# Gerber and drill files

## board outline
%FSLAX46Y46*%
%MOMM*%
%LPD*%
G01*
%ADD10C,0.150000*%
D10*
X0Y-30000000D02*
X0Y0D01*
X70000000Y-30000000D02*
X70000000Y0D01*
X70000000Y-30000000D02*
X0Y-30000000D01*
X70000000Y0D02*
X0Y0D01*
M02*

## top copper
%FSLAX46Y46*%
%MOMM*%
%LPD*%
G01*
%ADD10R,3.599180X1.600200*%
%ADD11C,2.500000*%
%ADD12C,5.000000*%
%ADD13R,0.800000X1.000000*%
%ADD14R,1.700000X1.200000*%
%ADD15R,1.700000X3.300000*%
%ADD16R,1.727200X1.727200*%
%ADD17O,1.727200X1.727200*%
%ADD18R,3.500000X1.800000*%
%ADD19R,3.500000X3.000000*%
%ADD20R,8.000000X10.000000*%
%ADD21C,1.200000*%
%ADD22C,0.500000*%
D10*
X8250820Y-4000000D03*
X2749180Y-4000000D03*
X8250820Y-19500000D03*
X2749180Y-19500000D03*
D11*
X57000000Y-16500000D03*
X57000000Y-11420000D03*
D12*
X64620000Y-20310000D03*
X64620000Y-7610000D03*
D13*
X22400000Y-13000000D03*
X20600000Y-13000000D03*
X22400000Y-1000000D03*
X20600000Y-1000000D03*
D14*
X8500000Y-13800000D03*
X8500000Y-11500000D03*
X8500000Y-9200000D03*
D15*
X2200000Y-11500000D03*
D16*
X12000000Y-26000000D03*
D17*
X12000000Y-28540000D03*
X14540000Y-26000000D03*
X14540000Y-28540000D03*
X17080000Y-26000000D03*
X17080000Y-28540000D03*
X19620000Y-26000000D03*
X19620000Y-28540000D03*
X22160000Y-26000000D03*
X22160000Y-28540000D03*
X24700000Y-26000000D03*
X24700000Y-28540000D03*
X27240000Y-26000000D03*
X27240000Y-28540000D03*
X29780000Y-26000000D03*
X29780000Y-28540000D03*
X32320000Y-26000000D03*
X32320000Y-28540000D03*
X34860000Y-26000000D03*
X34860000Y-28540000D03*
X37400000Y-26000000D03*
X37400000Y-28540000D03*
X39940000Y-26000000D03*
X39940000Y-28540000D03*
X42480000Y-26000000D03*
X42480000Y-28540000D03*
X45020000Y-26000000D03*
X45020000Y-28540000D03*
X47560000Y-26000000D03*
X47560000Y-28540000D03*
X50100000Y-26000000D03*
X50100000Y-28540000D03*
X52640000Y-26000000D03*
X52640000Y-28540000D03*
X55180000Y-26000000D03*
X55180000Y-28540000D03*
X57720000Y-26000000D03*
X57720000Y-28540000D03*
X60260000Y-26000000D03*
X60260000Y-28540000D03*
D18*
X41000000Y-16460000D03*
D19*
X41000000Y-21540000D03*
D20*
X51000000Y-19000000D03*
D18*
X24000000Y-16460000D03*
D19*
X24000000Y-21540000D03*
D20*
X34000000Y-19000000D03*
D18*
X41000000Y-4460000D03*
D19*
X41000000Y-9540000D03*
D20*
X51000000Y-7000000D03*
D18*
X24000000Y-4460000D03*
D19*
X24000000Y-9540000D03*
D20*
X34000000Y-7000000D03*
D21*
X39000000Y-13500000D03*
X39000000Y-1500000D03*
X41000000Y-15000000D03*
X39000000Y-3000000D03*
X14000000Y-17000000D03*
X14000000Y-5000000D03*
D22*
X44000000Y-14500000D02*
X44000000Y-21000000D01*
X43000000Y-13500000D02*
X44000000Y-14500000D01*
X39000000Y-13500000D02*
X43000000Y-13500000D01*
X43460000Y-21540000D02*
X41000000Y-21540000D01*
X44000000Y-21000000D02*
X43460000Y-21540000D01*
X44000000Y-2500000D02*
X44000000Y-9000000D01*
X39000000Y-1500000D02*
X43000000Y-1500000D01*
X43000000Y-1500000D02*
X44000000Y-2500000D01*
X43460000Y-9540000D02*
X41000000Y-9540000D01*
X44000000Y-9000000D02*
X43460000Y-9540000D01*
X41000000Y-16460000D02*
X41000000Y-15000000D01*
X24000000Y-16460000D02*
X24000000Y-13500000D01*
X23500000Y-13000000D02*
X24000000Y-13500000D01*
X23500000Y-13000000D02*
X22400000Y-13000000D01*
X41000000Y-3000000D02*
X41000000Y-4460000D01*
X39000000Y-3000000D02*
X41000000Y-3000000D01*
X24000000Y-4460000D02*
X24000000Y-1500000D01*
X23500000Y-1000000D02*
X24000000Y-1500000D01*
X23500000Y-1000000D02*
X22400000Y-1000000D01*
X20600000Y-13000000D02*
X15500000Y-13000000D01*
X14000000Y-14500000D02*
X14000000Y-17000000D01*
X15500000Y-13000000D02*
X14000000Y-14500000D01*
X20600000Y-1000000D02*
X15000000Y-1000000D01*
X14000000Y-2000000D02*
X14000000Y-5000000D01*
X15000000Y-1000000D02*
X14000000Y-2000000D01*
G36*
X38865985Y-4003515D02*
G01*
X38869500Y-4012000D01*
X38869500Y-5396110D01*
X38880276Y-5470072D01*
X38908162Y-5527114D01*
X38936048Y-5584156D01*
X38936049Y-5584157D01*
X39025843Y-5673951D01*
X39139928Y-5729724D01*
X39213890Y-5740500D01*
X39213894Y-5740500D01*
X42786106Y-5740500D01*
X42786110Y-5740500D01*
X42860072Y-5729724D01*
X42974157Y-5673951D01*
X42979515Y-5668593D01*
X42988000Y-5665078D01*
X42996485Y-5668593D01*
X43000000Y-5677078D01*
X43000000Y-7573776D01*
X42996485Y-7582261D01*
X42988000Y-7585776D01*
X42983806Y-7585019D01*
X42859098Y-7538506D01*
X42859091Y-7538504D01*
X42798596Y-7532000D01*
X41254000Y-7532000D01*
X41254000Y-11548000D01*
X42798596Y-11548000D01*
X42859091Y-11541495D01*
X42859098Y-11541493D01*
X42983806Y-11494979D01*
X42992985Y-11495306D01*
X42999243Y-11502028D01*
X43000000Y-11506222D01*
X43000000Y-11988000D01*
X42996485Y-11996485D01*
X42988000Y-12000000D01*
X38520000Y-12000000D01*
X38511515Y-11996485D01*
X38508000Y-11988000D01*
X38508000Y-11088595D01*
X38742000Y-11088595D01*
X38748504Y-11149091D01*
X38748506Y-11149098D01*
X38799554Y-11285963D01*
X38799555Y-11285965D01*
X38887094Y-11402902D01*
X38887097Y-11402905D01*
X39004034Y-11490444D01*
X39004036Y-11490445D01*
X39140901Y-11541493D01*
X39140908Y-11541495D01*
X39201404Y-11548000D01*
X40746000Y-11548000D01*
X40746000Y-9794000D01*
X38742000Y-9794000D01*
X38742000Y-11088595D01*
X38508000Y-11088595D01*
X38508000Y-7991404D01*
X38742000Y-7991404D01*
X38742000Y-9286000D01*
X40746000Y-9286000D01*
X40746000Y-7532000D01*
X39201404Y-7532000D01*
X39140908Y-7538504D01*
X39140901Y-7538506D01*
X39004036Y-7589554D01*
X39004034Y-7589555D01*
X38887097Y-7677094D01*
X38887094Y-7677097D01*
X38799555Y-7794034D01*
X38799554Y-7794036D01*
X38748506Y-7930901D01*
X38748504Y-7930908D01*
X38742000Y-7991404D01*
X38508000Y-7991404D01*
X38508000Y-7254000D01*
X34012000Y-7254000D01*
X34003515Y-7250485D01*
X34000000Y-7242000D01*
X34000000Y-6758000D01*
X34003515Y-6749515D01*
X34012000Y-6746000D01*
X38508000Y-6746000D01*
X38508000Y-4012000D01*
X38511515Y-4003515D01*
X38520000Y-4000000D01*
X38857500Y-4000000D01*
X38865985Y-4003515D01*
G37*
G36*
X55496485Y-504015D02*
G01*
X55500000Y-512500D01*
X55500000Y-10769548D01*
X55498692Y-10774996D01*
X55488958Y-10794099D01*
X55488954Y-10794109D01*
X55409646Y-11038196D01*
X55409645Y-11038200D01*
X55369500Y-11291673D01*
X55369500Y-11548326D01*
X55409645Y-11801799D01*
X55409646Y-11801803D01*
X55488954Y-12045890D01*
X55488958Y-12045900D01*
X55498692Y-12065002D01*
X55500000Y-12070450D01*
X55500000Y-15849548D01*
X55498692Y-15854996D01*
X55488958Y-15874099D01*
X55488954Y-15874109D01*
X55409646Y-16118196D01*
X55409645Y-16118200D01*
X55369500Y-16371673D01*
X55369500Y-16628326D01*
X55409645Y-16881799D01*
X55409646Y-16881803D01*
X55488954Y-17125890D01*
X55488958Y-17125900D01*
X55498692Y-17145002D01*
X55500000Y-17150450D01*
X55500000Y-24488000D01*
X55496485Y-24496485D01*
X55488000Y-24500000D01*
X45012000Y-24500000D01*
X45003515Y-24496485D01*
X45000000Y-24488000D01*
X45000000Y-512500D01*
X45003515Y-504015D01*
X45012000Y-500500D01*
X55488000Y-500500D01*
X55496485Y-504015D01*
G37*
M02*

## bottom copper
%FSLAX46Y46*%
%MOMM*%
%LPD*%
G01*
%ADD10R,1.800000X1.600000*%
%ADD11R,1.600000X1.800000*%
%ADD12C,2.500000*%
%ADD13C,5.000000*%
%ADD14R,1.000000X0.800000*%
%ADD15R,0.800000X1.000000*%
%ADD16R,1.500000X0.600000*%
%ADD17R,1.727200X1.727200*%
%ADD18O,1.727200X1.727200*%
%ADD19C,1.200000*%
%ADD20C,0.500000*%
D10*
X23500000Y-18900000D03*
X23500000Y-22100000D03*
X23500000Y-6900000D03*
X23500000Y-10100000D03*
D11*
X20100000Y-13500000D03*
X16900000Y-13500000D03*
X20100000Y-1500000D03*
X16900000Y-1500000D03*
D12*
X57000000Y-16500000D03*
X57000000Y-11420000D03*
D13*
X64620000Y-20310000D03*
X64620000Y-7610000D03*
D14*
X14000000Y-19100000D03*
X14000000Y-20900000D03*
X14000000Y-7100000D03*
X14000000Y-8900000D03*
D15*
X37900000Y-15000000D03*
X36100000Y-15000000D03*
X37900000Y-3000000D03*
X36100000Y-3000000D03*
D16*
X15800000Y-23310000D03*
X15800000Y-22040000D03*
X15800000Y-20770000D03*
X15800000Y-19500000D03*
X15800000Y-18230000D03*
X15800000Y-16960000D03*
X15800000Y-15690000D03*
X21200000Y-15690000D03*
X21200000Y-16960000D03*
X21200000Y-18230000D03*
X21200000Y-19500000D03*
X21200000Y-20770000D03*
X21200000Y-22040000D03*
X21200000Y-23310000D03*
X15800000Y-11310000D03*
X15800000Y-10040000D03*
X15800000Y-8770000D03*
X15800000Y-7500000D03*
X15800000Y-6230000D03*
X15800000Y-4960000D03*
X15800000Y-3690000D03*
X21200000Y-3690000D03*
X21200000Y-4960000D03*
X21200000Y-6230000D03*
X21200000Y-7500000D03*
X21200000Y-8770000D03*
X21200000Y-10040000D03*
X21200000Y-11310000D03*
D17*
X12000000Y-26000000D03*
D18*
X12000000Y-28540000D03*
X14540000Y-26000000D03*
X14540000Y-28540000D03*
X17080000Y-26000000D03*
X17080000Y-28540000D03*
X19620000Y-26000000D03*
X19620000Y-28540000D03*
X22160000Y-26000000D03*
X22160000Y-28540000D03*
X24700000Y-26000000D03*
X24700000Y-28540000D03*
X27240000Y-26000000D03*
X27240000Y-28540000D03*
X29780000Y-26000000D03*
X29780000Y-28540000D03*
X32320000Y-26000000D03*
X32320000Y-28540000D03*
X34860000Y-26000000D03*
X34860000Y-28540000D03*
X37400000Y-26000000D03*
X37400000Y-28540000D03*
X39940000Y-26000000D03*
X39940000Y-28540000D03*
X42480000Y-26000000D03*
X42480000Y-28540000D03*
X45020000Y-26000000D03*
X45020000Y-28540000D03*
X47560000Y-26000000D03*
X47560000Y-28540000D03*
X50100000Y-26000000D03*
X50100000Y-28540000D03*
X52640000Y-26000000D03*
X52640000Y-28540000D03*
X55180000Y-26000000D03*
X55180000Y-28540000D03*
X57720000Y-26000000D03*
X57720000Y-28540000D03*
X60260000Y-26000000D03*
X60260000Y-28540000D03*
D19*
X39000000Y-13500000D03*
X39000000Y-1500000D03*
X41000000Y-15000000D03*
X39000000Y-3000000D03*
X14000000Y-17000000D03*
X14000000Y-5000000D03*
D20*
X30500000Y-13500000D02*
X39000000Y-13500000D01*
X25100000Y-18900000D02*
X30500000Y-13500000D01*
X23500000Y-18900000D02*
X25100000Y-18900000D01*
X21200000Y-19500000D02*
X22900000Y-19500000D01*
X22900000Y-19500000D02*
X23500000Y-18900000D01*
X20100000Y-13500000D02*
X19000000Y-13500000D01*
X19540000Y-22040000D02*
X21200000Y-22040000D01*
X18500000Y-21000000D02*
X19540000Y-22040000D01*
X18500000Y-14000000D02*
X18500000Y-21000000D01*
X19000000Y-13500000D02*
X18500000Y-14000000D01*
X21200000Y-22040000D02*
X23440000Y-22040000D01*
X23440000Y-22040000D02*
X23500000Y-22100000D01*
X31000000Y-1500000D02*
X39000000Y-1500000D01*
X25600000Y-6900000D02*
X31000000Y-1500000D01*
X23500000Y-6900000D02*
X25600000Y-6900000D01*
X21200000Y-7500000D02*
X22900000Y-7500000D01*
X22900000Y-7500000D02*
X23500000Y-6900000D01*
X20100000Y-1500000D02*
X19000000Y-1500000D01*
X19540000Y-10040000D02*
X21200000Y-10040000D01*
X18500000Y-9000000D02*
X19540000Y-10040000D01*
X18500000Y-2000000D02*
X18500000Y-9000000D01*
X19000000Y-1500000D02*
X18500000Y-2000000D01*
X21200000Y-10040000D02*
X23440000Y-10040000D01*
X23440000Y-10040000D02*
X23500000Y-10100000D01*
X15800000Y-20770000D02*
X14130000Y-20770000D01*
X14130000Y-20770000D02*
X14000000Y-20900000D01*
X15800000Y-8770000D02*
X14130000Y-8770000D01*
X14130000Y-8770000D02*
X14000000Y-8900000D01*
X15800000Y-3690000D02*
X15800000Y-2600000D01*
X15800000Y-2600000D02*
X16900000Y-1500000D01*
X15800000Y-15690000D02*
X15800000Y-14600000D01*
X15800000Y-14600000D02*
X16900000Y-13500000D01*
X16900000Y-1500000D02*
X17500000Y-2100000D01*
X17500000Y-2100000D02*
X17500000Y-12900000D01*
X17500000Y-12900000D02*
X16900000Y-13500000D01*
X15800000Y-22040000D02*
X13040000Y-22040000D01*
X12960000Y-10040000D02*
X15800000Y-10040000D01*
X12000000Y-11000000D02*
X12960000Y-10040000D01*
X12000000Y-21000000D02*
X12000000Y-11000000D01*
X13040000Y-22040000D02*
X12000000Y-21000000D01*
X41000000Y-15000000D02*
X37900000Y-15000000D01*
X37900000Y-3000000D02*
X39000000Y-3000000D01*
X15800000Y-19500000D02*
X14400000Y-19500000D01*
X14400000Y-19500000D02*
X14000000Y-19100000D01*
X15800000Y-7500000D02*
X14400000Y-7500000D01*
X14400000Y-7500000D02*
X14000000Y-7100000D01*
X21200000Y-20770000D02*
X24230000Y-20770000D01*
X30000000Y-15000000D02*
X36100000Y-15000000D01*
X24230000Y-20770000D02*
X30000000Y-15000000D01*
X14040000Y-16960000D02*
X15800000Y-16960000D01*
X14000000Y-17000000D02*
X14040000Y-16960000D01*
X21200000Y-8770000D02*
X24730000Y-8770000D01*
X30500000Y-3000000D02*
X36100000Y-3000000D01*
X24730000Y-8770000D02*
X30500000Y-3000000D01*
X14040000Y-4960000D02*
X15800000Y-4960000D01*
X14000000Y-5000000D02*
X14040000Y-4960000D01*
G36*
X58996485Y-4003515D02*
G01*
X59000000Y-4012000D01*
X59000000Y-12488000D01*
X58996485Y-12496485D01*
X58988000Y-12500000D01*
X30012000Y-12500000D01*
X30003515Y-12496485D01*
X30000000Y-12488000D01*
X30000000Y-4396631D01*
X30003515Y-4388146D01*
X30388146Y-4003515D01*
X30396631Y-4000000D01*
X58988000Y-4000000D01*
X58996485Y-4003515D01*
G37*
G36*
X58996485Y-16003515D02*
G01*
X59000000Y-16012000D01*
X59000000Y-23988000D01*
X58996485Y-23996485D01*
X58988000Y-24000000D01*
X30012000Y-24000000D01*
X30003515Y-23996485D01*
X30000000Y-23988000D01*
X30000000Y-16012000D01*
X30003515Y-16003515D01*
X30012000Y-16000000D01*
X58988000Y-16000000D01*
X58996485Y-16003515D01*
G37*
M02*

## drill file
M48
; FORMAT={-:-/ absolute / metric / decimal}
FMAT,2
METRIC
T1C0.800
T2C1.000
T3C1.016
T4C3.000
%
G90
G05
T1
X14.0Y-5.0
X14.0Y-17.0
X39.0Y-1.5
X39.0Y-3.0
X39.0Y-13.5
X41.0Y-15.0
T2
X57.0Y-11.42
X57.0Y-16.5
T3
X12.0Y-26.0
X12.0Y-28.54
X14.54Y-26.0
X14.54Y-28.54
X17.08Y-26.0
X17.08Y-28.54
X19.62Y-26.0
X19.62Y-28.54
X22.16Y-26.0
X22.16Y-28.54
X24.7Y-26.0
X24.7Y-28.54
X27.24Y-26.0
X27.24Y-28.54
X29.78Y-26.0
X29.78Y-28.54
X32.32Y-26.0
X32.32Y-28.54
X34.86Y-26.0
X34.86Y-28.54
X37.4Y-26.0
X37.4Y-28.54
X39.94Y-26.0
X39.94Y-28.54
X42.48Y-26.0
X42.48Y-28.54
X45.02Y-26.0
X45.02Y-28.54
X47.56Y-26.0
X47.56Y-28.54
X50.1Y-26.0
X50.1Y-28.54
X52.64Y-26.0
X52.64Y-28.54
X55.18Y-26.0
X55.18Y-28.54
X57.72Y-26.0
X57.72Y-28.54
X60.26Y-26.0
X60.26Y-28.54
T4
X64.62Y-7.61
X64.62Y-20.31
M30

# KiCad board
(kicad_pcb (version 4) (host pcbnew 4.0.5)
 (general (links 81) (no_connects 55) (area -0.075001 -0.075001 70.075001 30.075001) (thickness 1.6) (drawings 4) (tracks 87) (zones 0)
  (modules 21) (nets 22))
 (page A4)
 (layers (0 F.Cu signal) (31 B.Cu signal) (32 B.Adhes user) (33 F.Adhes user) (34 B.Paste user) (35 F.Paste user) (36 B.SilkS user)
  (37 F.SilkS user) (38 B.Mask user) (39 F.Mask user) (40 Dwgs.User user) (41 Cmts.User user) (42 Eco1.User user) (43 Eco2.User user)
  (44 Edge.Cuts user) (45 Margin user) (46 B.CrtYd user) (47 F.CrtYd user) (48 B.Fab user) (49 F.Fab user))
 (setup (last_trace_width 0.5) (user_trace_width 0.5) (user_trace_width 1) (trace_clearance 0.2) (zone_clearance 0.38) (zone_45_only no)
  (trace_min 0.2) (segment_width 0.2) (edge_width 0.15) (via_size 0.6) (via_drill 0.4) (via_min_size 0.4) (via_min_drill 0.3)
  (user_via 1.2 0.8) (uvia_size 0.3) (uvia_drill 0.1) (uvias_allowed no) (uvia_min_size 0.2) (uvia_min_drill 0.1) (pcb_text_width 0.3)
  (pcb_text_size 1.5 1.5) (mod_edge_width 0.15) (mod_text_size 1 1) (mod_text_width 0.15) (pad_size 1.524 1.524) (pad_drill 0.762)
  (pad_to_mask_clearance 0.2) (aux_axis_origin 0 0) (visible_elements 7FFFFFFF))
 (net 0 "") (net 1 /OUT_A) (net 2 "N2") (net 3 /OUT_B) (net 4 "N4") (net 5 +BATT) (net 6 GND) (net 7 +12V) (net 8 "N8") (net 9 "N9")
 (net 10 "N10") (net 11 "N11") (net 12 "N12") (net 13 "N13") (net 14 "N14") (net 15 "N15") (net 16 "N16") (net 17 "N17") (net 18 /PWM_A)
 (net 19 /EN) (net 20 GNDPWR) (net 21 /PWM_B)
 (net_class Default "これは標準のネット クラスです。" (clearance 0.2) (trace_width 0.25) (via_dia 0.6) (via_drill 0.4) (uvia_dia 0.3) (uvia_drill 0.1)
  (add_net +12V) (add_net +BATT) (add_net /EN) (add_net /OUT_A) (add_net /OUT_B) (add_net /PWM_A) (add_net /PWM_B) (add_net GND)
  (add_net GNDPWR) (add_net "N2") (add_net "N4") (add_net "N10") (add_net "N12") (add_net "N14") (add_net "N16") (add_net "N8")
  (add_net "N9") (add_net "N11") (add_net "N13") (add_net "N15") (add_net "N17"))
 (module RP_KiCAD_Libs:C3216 (layer B.Cu) (at 23.5 20.5 270)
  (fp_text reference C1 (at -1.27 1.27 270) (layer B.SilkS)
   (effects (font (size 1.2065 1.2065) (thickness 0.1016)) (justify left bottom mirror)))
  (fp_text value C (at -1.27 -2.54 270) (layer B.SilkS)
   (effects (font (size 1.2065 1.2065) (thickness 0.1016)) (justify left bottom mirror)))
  (pad 1 smd rect (at -1.6 0 270) (size 1.6 1.8) (layers B.Cu B.Paste B.Mask) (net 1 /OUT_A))
  (pad 2 smd rect (at 1.6 0 270) (size 1.6 1.8) (layers B.Cu B.Paste B.Mask) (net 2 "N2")))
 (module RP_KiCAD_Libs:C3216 (layer B.Cu) (at 23.5 8.5 270)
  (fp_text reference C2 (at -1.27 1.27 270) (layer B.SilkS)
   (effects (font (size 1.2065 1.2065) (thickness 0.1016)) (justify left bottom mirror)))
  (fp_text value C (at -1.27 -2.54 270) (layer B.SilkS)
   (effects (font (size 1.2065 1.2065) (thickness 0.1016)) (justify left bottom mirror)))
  (pad 1 smd rect (at -1.6 0 270) (size 1.6 1.8) (layers B.Cu B.Paste B.Mask) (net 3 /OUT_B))
  (pad 2 smd rect (at 1.6 0 270) (size 1.6 1.8) (layers B.Cu B.Paste B.Mask) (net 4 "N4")))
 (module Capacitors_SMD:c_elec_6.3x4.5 (layer F.Cu) (at 5.5 4)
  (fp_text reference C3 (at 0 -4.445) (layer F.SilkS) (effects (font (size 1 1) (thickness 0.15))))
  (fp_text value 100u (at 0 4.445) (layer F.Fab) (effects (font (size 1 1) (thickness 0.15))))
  (pad 1 smd rect (at 2.75082 0) (size 3.59918 1.6002) (layers F.Cu F.Paste F.Mask) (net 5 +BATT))
  (pad 2 smd rect (at -2.75082 0) (size 3.59918 1.6002) (layers F.Cu F.Paste F.Mask) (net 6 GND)))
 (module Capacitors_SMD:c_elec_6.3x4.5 (layer F.Cu) (at 5.5 19.5)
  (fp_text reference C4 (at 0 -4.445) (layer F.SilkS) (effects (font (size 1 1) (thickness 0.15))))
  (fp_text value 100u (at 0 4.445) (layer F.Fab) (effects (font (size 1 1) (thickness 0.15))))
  (pad 1 smd rect (at 2.75082 0) (size 3.59918 1.6002) (layers F.Cu F.Paste F.Mask) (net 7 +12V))
  (pad 2 smd rect (at -2.75082 0) (size 3.59918 1.6002) (layers F.Cu F.Paste F.Mask) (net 6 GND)))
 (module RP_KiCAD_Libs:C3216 (layer B.Cu) (at 18.5 13.5 180)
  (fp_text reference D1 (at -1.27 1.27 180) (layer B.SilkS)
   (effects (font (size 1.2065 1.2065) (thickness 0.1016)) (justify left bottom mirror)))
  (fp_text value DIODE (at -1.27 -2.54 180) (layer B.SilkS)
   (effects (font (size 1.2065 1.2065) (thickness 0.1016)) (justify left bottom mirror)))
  (pad 1 smd rect (at -1.6 0 180) (size 1.6 1.8) (layers B.Cu B.Paste B.Mask) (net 2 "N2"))
  (pad 2 smd rect (at 1.6 0 180) (size 1.6 1.8) (layers B.Cu B.Paste B.Mask) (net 7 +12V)))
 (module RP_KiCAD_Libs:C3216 (layer B.Cu) (at 18.5 1.5 180)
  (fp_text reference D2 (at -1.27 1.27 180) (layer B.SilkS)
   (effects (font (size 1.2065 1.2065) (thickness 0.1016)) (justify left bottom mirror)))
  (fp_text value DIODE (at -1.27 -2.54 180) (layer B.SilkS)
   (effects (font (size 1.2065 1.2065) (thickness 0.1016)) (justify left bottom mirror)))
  (pad 1 smd rect (at -1.6 0 180) (size 1.6 1.8) (layers B.Cu B.Paste B.Mask) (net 4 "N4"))
  (pad 2 smd rect (at 1.6 0 180) (size 1.6 1.8) (layers B.Cu B.Paste B.Mask) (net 7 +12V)))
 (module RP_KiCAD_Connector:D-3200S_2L (layer F.Cu) (at 57 16.5 90)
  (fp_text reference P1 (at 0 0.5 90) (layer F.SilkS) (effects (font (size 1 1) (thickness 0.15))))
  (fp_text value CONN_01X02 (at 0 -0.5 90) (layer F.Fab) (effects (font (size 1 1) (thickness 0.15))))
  (pad 1 thru_hole circle (at 0 0 90) (size 2.5 2.5) (drill 1) (layers *.Cu *.Mask F.SilkS) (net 1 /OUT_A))
  (pad 2 thru_hole circle (at 5.08 0 90) (size 2.5 2.5) (drill 1) (layers *.Cu *.Mask F.SilkS) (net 3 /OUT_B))
  (pad "" thru_hole circle (at -3.81 7.62 90) (size 5 5) (drill 3) (layers *.Cu *.Mask F.SilkS))
  (pad "" thru_hole circle (at 8.89 7.62 90) (size 5 5) (drill 3) (layers *.Cu *.Mask F.SilkS)))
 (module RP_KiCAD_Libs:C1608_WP (layer B.Cu) (at 14 20 270)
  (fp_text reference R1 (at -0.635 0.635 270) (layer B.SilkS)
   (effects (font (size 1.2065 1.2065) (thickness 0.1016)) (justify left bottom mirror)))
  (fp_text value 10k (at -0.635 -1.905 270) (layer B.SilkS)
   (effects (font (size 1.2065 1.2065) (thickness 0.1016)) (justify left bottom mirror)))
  (pad 1 smd rect (at -0.9 0 270) (size 0.8 1) (layers B.Cu B.Paste B.Mask) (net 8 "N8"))
  (pad 2 smd rect (at 0.9 0 270) (size 0.8 1) (layers B.Cu B.Paste B.Mask) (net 6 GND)))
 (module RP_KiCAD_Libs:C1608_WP (layer B.Cu) (at 14 8 270)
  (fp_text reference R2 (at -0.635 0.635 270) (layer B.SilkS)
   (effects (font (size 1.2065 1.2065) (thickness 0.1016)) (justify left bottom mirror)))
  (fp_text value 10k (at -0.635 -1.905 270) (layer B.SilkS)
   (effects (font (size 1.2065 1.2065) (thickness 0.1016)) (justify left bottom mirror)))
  (pad 1 smd rect (at -0.9 0 270) (size 0.8 1) (layers B.Cu B.Paste B.Mask) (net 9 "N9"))
  (pad 2 smd rect (at 0.9 0 270) (size 0.8 1) (layers B.Cu B.Paste B.Mask) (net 6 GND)))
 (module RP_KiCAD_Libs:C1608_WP (layer B.Cu) (at 37 15 180)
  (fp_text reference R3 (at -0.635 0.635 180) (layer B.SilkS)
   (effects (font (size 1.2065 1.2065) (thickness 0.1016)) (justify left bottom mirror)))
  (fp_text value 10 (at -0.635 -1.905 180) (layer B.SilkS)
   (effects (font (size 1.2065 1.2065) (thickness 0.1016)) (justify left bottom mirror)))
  (pad 1 smd rect (at -0.9 0 180) (size 0.8 1) (layers B.Cu B.Paste B.Mask) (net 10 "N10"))
  (pad 2 smd rect (at 0.9 0 180) (size 0.8 1) (layers B.Cu B.Paste B.Mask) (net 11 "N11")))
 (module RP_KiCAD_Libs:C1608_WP (layer F.Cu) (at 21.5 13 180)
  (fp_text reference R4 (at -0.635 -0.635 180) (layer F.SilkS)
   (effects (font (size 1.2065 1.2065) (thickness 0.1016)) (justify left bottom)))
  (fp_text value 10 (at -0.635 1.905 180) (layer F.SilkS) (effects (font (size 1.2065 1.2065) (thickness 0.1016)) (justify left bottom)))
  (pad 1 smd rect (at -0.9 0 180) (size 0.8 1) (layers F.Cu F.Paste F.Mask) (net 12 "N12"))
  (pad 2 smd rect (at 0.9 0 180) (size 0.8 1) (layers F.Cu F.Paste F.Mask) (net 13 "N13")))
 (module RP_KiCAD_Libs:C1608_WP (layer B.Cu) (at 37 3 180)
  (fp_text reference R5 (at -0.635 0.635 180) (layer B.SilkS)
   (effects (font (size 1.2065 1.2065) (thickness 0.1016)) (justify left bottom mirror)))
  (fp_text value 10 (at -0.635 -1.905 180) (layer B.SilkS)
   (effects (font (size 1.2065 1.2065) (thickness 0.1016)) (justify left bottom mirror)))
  (pad 1 smd rect (at -0.9 0 180) (size 0.8 1) (layers B.Cu B.Paste B.Mask) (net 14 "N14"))
  (pad 2 smd rect (at 0.9 0 180) (size 0.8 1) (layers B.Cu B.Paste B.Mask) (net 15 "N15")))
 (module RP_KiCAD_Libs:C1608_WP (layer F.Cu) (at 21.5 1 180)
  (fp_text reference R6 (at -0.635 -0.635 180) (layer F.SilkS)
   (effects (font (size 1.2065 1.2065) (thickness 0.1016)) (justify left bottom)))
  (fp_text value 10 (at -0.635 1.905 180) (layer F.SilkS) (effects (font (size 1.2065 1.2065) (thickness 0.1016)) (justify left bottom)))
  (pad 1 smd rect (at -0.9 0 180) (size 0.8 1) (layers F.Cu F.Paste F.Mask) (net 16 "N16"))
  (pad 2 smd rect (at 0.9 0 180) (size 0.8 1) (layers F.Cu F.Paste F.Mask) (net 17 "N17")))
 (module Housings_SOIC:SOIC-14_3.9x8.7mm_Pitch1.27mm (layer B.Cu) (at 18.5 19.5)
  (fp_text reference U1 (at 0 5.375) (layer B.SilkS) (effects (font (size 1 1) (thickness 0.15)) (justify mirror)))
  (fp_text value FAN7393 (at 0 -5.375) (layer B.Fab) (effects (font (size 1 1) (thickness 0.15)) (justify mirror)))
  (pad 1 smd rect (at -2.7 3.81) (size 1.5 0.6) (layers B.Cu B.Paste B.Mask) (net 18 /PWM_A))
  (pad 2 smd rect (at -2.7 2.54) (size 1.5 0.6) (layers B.Cu B.Paste B.Mask) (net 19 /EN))
  (pad 3 smd rect (at -2.7 1.27) (size 1.5 0.6) (layers B.Cu B.Paste B.Mask) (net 6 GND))
  (pad 4 smd rect (at -2.7 0) (size 1.5 0.6) (layers B.Cu B.Paste B.Mask) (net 8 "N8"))
  (pad 5 smd rect (at -2.7 -1.27) (size 1.5 0.6) (layers B.Cu B.Paste B.Mask) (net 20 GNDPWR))
  (pad 6 smd rect (at -2.7 -2.54) (size 1.5 0.6) (layers B.Cu B.Paste B.Mask) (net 13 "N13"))
  (pad 7 smd rect (at -2.7 -3.81) (size 1.5 0.6) (layers B.Cu B.Paste B.Mask) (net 7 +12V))
  (pad 8 smd rect (at 2.7 -3.81) (size 1.5 0.6) (layers B.Cu B.Paste B.Mask))
  (pad 9 smd rect (at 2.7 -2.54) (size 1.5 0.6) (layers B.Cu B.Paste B.Mask))
  (pad 10 smd rect (at 2.7 -1.27) (size 1.5 0.6) (layers B.Cu B.Paste B.Mask))
  (pad 11 smd rect (at 2.7 0) (size 1.5 0.6) (layers B.Cu B.Paste B.Mask) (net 1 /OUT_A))
  (pad 12 smd rect (at 2.7 1.27) (size 1.5 0.6) (layers B.Cu B.Paste B.Mask) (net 11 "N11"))
  (pad 13 smd rect (at 2.7 2.54) (size 1.5 0.6) (layers B.Cu B.Paste B.Mask) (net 2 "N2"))
  (pad 14 smd rect (at 2.7 3.81) (size 1.5 0.6) (layers B.Cu B.Paste B.Mask)))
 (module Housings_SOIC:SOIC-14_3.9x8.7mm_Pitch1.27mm (layer B.Cu) (at 18.5 7.5)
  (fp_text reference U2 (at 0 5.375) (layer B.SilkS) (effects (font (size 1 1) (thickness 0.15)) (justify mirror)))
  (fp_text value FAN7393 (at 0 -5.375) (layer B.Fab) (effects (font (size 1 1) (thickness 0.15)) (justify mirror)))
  (pad 1 smd rect (at -2.7 3.81) (size 1.5 0.6) (layers B.Cu B.Paste B.Mask) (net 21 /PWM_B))
  (pad 2 smd rect (at -2.7 2.54) (size 1.5 0.6) (layers B.Cu B.Paste B.Mask) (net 19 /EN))
  (pad 3 smd rect (at -2.7 1.27) (size 1.5 0.6) (layers B.Cu B.Paste B.Mask) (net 6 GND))
  (pad 4 smd rect (at -2.7 0) (size 1.5 0.6) (layers B.Cu B.Paste B.Mask) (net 9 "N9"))
  (pad 5 smd rect (at -2.7 -1.27) (size 1.5 0.6) (layers B.Cu B.Paste B.Mask) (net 20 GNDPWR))
  (pad 6 smd rect (at -2.7 -2.54) (size 1.5 0.6) (layers B.Cu B.Paste B.Mask) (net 17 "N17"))
  (pad 7 smd rect (at -2.7 -3.81) (size 1.5 0.6) (layers B.Cu B.Paste B.Mask) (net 7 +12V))
  (pad 8 smd rect (at 2.7 -3.81) (size 1.5 0.6) (layers B.Cu B.Paste B.Mask))
  (pad 9 smd rect (at 2.7 -2.54) (size 1.5 0.6) (layers B.Cu B.Paste B.Mask))
  (pad 10 smd rect (at 2.7 -1.27) (size 1.5 0.6) (layers B.Cu B.Paste B.Mask))
  (pad 11 smd rect (at 2.7 0) (size 1.5 0.6) (layers B.Cu B.Paste B.Mask) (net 3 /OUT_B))
  (pad 12 smd rect (at 2.7 1.27) (size 1.5 0.6) (layers B.Cu B.Paste B.Mask) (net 15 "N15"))
  (pad 13 smd rect (at 2.7 2.54) (size 1.5 0.6) (layers B.Cu B.Paste B.Mask) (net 4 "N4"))
  (pad 14 smd rect (at 2.7 3.81) (size 1.5 0.6) (layers B.Cu B.Paste B.Mask)))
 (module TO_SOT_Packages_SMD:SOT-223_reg (layer F.Cu) (at 8.5 11.5 90)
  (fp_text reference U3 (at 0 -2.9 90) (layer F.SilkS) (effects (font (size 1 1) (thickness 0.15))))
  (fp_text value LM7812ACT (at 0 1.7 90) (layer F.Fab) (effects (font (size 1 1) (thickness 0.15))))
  (pad 1 smd rect (at -2.3 0 90) (size 1.2 1.7) (layers F.Cu F.Paste F.Mask) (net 5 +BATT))
  (pad 2 smd rect (at 0 0 90) (size 1.2 1.7) (layers F.Cu F.Paste F.Mask) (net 6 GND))
  (pad 3 smd rect (at 2.3 0 90) (size 1.2 1.7) (layers F.Cu F.Paste F.Mask) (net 7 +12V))
  (pad 2 smd rect (at 0 -6.3 90) (size 3.3 1.7) (layers F.Cu F.Paste F.Mask) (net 6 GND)))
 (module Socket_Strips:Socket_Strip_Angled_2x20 (layer F.Cu) (at 12 26)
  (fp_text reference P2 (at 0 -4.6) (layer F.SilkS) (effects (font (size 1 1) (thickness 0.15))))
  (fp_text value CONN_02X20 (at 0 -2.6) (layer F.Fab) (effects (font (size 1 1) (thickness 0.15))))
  (pad 1 thru_hole rect (at 0 0) (size 1.7272 1.7272) (drill 1.016) (layers *.Cu *.Mask F.SilkS) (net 6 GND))
  (pad 2 thru_hole oval (at 0 2.54) (size 1.7272 1.7272) (drill 1.016) (layers *.Cu *.Mask F.SilkS) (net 21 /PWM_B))
  (pad 3 thru_hole oval (at 2.54 0) (size 1.7272 1.7272) (drill 1.016) (layers *.Cu *.Mask F.SilkS) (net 19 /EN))
  (pad 4 thru_hole oval (at 2.54 2.54) (size 1.7272 1.7272) (drill 1.016) (layers *.Cu *.Mask F.SilkS) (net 18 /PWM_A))
  (pad 5 thru_hole oval (at 5.08 0) (size 1.7272 1.7272) (drill 1.016) (layers *.Cu *.Mask F.SilkS) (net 20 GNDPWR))
  (pad 6 thru_hole oval (at 5.08 2.54) (size 1.7272 1.7272) (drill 1.016) (layers *.Cu *.Mask F.SilkS) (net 20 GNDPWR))
  (pad 7 thru_hole oval (at 7.62 0) (size 1.7272 1.7272) (drill 1.016) (layers *.Cu *.Mask F.SilkS) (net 20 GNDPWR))
  (pad 8 thru_hole oval (at 7.62 2.54) (size 1.7272 1.7272) (drill 1.016) (layers *.Cu *.Mask F.SilkS) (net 20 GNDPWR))
  (pad 9 thru_hole oval (at 10.16 0) (size 1.7272 1.7272) (drill 1.016) (layers *.Cu *.Mask F.SilkS) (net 20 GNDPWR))
  (pad 10 thru_hole oval (at 10.16 2.54) (size 1.7272 1.7272) (drill 1.016) (layers *.Cu *.Mask F.SilkS) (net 20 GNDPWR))
  (pad 11 thru_hole oval (at 12.7 0) (size 1.7272 1.7272) (drill 1.016) (layers *.Cu *.Mask F.SilkS) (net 20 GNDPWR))
  (pad 12 thru_hole oval (at 12.7 2.54) (size 1.7272 1.7272) (drill 1.016) (layers *.Cu *.Mask F.SilkS) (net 20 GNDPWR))
  (pad 13 thru_hole oval (at 15.24 0) (size 1.7272 1.7272) (drill 1.016) (layers *.Cu *.Mask F.SilkS) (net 20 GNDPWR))
  (pad 14 thru_hole oval (at 15.24 2.54) (size 1.7272 1.7272) (drill 1.016) (layers *.Cu *.Mask F.SilkS) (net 20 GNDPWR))
  (pad 15 thru_hole oval (at 17.78 0) (size 1.7272 1.7272) (drill 1.016) (layers *.Cu *.Mask F.SilkS) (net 20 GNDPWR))
  (pad 16 thru_hole oval (at 17.78 2.54) (size 1.7272 1.7272) (drill 1.016) (layers *.Cu *.Mask F.SilkS) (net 20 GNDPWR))
  (pad 17 thru_hole oval (at 20.32 0) (size 1.7272 1.7272) (drill 1.016) (layers *.Cu *.Mask F.SilkS) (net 20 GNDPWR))
  (pad 18 thru_hole oval (at 20.32 2.54) (size 1.7272 1.7272) (drill 1.016) (layers *.Cu *.Mask F.SilkS) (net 20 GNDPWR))
  (pad 19 thru_hole oval (at 22.86 0) (size 1.7272 1.7272) (drill 1.016) (layers *.Cu *.Mask F.SilkS) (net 20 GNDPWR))
  (pad 20 thru_hole oval (at 22.86 2.54) (size 1.7272 1.7272) (drill 1.016) (layers *.Cu *.Mask F.SilkS) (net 20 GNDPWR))
  (pad 21 thru_hole oval (at 25.4 0) (size 1.7272 1.7272) (drill 1.016) (layers *.Cu *.Mask F.SilkS) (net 20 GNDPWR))
  (pad 22 thru_hole oval (at 25.4 2.54) (size 1.7272 1.7272) (drill 1.016) (layers *.Cu *.Mask F.SilkS) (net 20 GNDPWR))
  (pad 23 thru_hole oval (at 27.94 0) (size 1.7272 1.7272) (drill 1.016) (layers *.Cu *.Mask F.SilkS) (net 5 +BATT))
  (pad 24 thru_hole oval (at 27.94 2.54) (size 1.7272 1.7272) (drill 1.016) (layers *.Cu *.Mask F.SilkS) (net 5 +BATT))
  (pad 25 thru_hole oval (at 30.48 0) (size 1.7272 1.7272) (drill 1.016) (layers *.Cu *.Mask F.SilkS) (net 5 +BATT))
  (pad 26 thru_hole oval (at 30.48 2.54) (size 1.7272 1.7272) (drill 1.016) (layers *.Cu *.Mask F.SilkS) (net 5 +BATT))
  (pad 27 thru_hole oval (at 33.02 0) (size 1.7272 1.7272) (drill 1.016) (layers *.Cu *.Mask F.SilkS) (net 5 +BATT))
  (pad 28 thru_hole oval (at 33.02 2.54) (size 1.7272 1.7272) (drill 1.016) (layers *.Cu *.Mask F.SilkS) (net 5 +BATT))
  (pad 29 thru_hole oval (at 35.56 0) (size 1.7272 1.7272) (drill 1.016) (layers *.Cu *.Mask F.SilkS) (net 5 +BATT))
  (pad 30 thru_hole oval (at 35.56 2.54) (size 1.7272 1.7272) (drill 1.016) (layers *.Cu *.Mask F.SilkS) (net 5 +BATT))
  (pad 31 thru_hole oval (at 38.1 0) (size 1.7272 1.7272) (drill 1.016) (layers *.Cu *.Mask F.SilkS) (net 5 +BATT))
  (pad 32 thru_hole oval (at 38.1 2.54) (size 1.7272 1.7272) (drill 1.016) (layers *.Cu *.Mask F.SilkS) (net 5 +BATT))
  (pad 33 thru_hole oval (at 40.64 0) (size 1.7272 1.7272) (drill 1.016) (layers *.Cu *.Mask F.SilkS) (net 5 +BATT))
  (pad 34 thru_hole oval (at 40.64 2.54) (size 1.7272 1.7272) (drill 1.016) (layers *.Cu *.Mask F.SilkS) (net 5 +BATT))
  (pad 35 thru_hole oval (at 43.18 0) (size 1.7272 1.7272) (drill 1.016) (layers *.Cu *.Mask F.SilkS) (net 5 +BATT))
  (pad 36 thru_hole oval (at 43.18 2.54) (size 1.7272 1.7272) (drill 1.016) (layers *.Cu *.Mask F.SilkS) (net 5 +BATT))
  (pad 37 thru_hole oval (at 45.72 0) (size 1.7272 1.7272) (drill 1.016) (layers *.Cu *.Mask F.SilkS) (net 5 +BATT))
  (pad 38 thru_hole oval (at 45.72 2.54) (size 1.7272 1.7272) (drill 1.016) (layers *.Cu *.Mask F.SilkS) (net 5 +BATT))
  (pad 39 thru_hole oval (at 48.26 0) (size 1.7272 1.7272) (drill 1.016) (layers *.Cu *.Mask F.SilkS) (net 5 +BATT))
  (pad 40 thru_hole oval (at 48.26 2.54) (size 1.7272 1.7272) (drill 1.016) (layers *.Cu *.Mask F.SilkS) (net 5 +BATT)))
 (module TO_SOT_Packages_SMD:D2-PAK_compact (layer F.Cu) (at 44 19 270)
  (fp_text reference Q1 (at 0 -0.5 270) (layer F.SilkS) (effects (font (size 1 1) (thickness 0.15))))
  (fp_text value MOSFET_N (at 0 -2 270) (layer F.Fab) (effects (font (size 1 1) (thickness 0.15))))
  (pad G smd rect (at -2.54 3 270) (size 1.8 3.5) (layers F.Cu F.Paste F.Mask) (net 10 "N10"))
  (pad S smd rect (at 2.54 3 270) (size 3 3.5) (layers F.Cu F.Paste F.Mask) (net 1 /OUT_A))
  (pad D smd rect (at 0 -7 270) (size 10 8) (layers F.Cu F.Paste F.Mask) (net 5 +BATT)))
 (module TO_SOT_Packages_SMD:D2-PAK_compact (layer F.Cu) (at 27 19 270)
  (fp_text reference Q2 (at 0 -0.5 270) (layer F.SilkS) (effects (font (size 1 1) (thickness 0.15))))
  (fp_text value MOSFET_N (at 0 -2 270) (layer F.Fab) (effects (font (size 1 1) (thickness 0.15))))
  (pad G smd rect (at -2.54 3 270) (size 1.8 3.5) (layers F.Cu F.Paste F.Mask) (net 12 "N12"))
  (pad S smd rect (at 2.54 3 270) (size 3 3.5) (layers F.Cu F.Paste F.Mask) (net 20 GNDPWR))
  (pad D smd rect (at 0 -7 270) (size 10 8) (layers F.Cu F.Paste F.Mask) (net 1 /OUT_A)))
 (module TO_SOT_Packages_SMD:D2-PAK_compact (layer F.Cu) (at 44 7 270)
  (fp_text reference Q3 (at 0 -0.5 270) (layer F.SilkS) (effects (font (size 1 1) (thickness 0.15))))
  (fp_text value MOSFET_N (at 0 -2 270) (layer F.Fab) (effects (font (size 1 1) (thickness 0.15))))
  (pad G smd rect (at -2.54 3 270) (size 1.8 3.5) (layers F.Cu F.Paste F.Mask) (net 14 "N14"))
  (pad S smd rect (at 2.54 3 270) (size 3 3.5) (layers F.Cu F.Paste F.Mask) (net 3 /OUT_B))
  (pad D smd rect (at 0 -7 270) (size 10 8) (layers F.Cu F.Paste F.Mask) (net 5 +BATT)))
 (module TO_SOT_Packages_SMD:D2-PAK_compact (layer F.Cu) (at 27 7 270)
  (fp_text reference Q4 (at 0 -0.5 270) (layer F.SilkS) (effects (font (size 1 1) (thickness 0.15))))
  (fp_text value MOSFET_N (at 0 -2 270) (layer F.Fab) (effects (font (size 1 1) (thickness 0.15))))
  (pad G smd rect (at -2.54 3 270) (size 1.8 3.5) (layers F.Cu F.Paste F.Mask) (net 16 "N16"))
  (pad S smd rect (at 2.54 3 270) (size 3 3.5) (layers F.Cu F.Paste F.Mask) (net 20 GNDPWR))
  (pad D smd rect (at 0 -7 270) (size 10 8) (layers F.Cu F.Paste F.Mask) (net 3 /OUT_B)))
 (gr_line (start 0 30) (end 0 0) (angle 90) (layer Edge.Cuts) (width 0.15))
 (gr_line (start 70 30) (end 70 0) (angle 90) (layer Edge.Cuts) (width 0.15))
 (gr_line (start 70 30) (end 0 30) (angle 90) (layer Edge.Cuts) (width 0.15))
 (gr_line (start 70 0) (end 0 0) (angle 90) (layer Edge.Cuts) (width 0.15))
 (segment (start 44 14.5) (end 44 21) (width 0.5) (layer F.Cu) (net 1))
 (segment (start 43 13.5) (end 44 14.5) (width 0.5) (layer F.Cu) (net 1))
 (segment (start 39 13.5) (end 43 13.5) (width 0.5) (layer F.Cu) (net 1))
 (via (at 39 13.5) (size 1.2) (drill 0.8) (layers F.Cu B.Cu) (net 1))
 (segment (start 30.5 13.5) (end 39 13.5) (width 0.5) (layer B.Cu) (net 1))
 (segment (start 25.1 18.9) (end 30.5 13.5) (width 0.5) (layer B.Cu) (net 1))
 (segment (start 23.5 18.9) (end 25.1 18.9) (width 0.5) (layer B.Cu) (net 1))
 (segment (start 43.46 21.54) (end 41 21.54) (width 0.5) (layer F.Cu) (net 1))
 (segment (start 44 21) (end 43.46 21.54) (width 0.5) (layer F.Cu) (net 1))
 (segment (start 21.2 19.5) (end 22.9 19.5) (width 0.5) (layer B.Cu) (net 1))
 (segment (start 22.9 19.5) (end 23.5 18.9) (width 0.5) (layer B.Cu) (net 1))
 (segment (start 20.1 13.5) (end 19 13.5) (width 0.5) (layer B.Cu) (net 2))
 (segment (start 19.54 22.04) (end 21.2 22.04) (width 0.5) (layer B.Cu) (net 2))
 (segment (start 18.5 21) (end 19.54 22.04) (width 0.5) (layer B.Cu) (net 2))
 (segment (start 18.5 14) (end 18.5 21) (width 0.5) (layer B.Cu) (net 2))
 (segment (start 19 13.5) (end 18.5 14) (width 0.5) (layer B.Cu) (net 2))
 (segment (start 21.2 22.04) (end 23.44 22.04) (width 0.5) (layer B.Cu) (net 2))
 (segment (start 23.44 22.04) (end 23.5 22.1) (width 0.5) (layer B.Cu) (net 2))
 (segment (start 44 2.5) (end 44 9) (width 0.5) (layer F.Cu) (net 3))
 (via (at 39 1.5) (size 1.2) (drill 0.8) (layers F.Cu B.Cu) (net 3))
 (segment (start 39 1.5) (end 43 1.5) (width 0.5) (layer F.Cu) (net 3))
 (segment (start 43 1.5) (end 44 2.5) (width 0.5) (layer F.Cu) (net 3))
 (segment (start 31 1.5) (end 39 1.5) (width 0.5) (layer B.Cu) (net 3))
 (segment (start 25.6 6.9) (end 31 1.5) (width 0.5) (layer B.Cu) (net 3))
 (segment (start 23.5 6.9) (end 25.6 6.9) (width 0.5) (layer B.Cu) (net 3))
 (segment (start 43.46 9.54) (end 41 9.54) (width 0.5) (layer F.Cu) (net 3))
 (segment (start 44 9) (end 43.46 9.54) (width 0.5) (layer F.Cu) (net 3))
 (segment (start 21.2 7.5) (end 22.9 7.5) (width 0.5) (layer B.Cu) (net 3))
 (segment (start 22.9 7.5) (end 23.5 6.9) (width 0.5) (layer B.Cu) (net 3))
 (segment (start 20.1 1.5) (end 19 1.5) (width 0.5) (layer B.Cu) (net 4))
 (segment (start 19.54 10.04) (end 21.2 10.04) (width 0.5) (layer B.Cu) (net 4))
 (segment (start 18.5 9) (end 19.54 10.04) (width 0.5) (layer B.Cu) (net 4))
 (segment (start 18.5 2) (end 18.5 9) (width 0.5) (layer B.Cu) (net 4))
 (segment (start 19 1.5) (end 18.5 2) (width 0.5) (layer B.Cu) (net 4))
 (segment (start 21.2 10.04) (end 23.44 10.04) (width 0.5) (layer B.Cu) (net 4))
 (segment (start 23.44 10.04) (end 23.5 10.1) (width 0.5) (layer B.Cu) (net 4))
 (segment (start 15.8 20.77) (end 14.13 20.77) (width 0.5) (layer B.Cu) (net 6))
 (segment (start 14.13 20.77) (end 14 20.9) (width 0.5) (layer B.Cu) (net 6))
 (segment (start 15.8 8.77) (end 14.13 8.77) (width 0.5) (layer B.Cu) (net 6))
 (segment (start 14.13 8.77) (end 14 8.9) (width 0.5) (layer B.Cu) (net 6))
 (segment (start 15.8 3.69) (end 15.8 2.6) (width 0.5) (layer B.Cu) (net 7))
 (segment (start 15.8 2.6) (end 16.9 1.5) (width 0.5) (layer B.Cu) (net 7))
 (segment (start 15.8 15.69) (end 15.8 14.6) (width 0.5) (layer B.Cu) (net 7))
 (segment (start 15.8 14.6) (end 16.9 13.5) (width 0.5) (layer B.Cu) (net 7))
 (segment (start 16.9 1.5) (end 17.5 2.1) (width 0.5) (layer B.Cu) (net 7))
 (segment (start 17.5 2.1) (end 17.5 12.9) (width 0.5) (layer B.Cu) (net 7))
 (segment (start 17.5 12.9) (end 16.9 13.5) (width 0.5) (layer B.Cu) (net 7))
 (segment (start 15.8 22.04) (end 13.04 22.04) (width 0.5) (layer B.Cu) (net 19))
 (segment (start 12.96 10.04) (end 15.8 10.04) (width 0.5) (layer B.Cu) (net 19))
 (segment (start 12 11) (end 12.96 10.04) (width 0.5) (layer B.Cu) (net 19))
 (segment (start 12 21) (end 12 11) (width 0.5) (layer B.Cu) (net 19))
 (segment (start 13.04 22.04) (end 12 21) (width 0.5) (layer B.Cu) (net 19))
 (segment (start 41 16.46) (end 41 15) (width 0.5) (layer F.Cu) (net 10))
 (segment (start 41 15) (end 37.9 15) (width 0.5) (layer B.Cu) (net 10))
 (via (at 41 15) (size 1.2) (drill 0.8) (layers F.Cu B.Cu) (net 10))
 (segment (start 24 16.46) (end 24 13.5) (width 0.5) (layer F.Cu) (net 12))
 (segment (start 23.5 13) (end 24 13.5) (width 0.5) (layer F.Cu) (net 12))
 (segment (start 23.5 13) (end 22.4 13) (width 0.5) (layer F.Cu) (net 12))
 (segment (start 37.9 3) (end 39 3) (width 0.5) (layer B.Cu) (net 14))
 (segment (start 41 3) (end 41 4.46) (width 0.5) (layer F.Cu) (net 14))
 (segment (start 39 3) (end 41 3) (width 0.5) (layer F.Cu) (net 14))
 (via (at 39 3) (size 1.2) (drill 0.8) (layers F.Cu B.Cu) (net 14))
 (segment (start 24 4.46) (end 24 1.5) (width 0.5) (layer F.Cu) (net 16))
 (segment (start 23.5 1) (end 24 1.5) (width 0.5) (layer F.Cu) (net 16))
 (segment (start 23.5 1) (end 22.4 1) (width 0.5) (layer F.Cu) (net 16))
 (segment (start 15.8 19.5) (end 14.4 19.5) (width 0.5) (layer B.Cu) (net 8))
 (segment (start 14.4 19.5) (end 14 19.1) (width 0.5) (layer B.Cu) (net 8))
 (segment (start 15.8 7.5) (end 14.4 7.5) (width 0.5) (layer B.Cu) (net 9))
 (segment (start 14.4 7.5) (end 14 7.1) (width 0.5) (layer B.Cu) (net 9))
 (segment (start 21.2 20.77) (end 24.23 20.77) (width 0.5) (layer B.Cu) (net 11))
 (segment (start 30 15) (end 36.1 15) (width 0.5) (layer B.Cu) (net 11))
 (segment (start 24.23 20.77) (end 30 15) (width 0.5) (layer B.Cu) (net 11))
 (segment (start 20.6 13) (end 15.5 13) (width 0.5) (layer F.Cu) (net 13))
 (segment (start 14.04 16.96) (end 15.8 16.96) (width 0.5) (layer B.Cu) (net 13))
 (segment (start 14 17) (end 14.04 16.96) (width 0.5) (layer B.Cu) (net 13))
 (via (at 14 17) (size 1.2) (drill 0.8) (layers F.Cu B.Cu) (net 13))
 (segment (start 14 14.5) (end 14 17) (width 0.5) (layer F.Cu) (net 13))
 (segment (start 15.5 13) (end 14 14.5) (width 0.5) (layer F.Cu) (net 13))
 (segment (start 21.2 8.77) (end 24.73 8.77) (width 0.5) (layer B.Cu) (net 15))
 (segment (start 30.5 3) (end 36.1 3) (width 0.5) (layer B.Cu) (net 15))
 (segment (start 24.73 8.77) (end 30.5 3) (width 0.5) (layer B.Cu) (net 15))
 (segment (start 20.6 1) (end 15 1) (width 0.5) (layer F.Cu) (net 17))
 (segment (start 14.04 4.96) (end 15.8 4.96) (width 0.5) (layer B.Cu) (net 17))
 (segment (start 14 5) (end 14.04 4.96) (width 0.5) (layer B.Cu) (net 17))
 (via (at 14 5) (size 1.2) (drill 0.8) (layers F.Cu B.Cu) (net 17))
 (segment (start 14 2) (end 14 5) (width 0.5) (layer F.Cu) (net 17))
 (segment (start 15 1) (end 14 2) (width 0.5) (layer F.Cu) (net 17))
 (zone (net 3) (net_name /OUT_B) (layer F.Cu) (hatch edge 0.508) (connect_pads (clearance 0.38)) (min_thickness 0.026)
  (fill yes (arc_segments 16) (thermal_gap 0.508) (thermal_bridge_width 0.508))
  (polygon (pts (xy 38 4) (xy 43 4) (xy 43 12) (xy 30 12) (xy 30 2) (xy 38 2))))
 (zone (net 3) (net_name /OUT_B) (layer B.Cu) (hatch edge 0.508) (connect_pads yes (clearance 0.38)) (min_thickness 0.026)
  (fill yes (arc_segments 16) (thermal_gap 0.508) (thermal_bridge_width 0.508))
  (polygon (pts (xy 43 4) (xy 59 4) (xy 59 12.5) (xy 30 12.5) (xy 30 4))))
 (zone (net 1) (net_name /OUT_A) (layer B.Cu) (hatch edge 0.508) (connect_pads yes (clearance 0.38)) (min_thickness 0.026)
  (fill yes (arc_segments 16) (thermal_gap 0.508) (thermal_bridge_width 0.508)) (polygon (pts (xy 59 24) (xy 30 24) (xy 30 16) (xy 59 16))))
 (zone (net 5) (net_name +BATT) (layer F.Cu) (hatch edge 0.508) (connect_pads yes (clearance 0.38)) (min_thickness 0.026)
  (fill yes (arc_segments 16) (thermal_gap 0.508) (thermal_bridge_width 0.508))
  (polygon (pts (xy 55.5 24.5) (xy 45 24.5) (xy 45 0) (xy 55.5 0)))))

